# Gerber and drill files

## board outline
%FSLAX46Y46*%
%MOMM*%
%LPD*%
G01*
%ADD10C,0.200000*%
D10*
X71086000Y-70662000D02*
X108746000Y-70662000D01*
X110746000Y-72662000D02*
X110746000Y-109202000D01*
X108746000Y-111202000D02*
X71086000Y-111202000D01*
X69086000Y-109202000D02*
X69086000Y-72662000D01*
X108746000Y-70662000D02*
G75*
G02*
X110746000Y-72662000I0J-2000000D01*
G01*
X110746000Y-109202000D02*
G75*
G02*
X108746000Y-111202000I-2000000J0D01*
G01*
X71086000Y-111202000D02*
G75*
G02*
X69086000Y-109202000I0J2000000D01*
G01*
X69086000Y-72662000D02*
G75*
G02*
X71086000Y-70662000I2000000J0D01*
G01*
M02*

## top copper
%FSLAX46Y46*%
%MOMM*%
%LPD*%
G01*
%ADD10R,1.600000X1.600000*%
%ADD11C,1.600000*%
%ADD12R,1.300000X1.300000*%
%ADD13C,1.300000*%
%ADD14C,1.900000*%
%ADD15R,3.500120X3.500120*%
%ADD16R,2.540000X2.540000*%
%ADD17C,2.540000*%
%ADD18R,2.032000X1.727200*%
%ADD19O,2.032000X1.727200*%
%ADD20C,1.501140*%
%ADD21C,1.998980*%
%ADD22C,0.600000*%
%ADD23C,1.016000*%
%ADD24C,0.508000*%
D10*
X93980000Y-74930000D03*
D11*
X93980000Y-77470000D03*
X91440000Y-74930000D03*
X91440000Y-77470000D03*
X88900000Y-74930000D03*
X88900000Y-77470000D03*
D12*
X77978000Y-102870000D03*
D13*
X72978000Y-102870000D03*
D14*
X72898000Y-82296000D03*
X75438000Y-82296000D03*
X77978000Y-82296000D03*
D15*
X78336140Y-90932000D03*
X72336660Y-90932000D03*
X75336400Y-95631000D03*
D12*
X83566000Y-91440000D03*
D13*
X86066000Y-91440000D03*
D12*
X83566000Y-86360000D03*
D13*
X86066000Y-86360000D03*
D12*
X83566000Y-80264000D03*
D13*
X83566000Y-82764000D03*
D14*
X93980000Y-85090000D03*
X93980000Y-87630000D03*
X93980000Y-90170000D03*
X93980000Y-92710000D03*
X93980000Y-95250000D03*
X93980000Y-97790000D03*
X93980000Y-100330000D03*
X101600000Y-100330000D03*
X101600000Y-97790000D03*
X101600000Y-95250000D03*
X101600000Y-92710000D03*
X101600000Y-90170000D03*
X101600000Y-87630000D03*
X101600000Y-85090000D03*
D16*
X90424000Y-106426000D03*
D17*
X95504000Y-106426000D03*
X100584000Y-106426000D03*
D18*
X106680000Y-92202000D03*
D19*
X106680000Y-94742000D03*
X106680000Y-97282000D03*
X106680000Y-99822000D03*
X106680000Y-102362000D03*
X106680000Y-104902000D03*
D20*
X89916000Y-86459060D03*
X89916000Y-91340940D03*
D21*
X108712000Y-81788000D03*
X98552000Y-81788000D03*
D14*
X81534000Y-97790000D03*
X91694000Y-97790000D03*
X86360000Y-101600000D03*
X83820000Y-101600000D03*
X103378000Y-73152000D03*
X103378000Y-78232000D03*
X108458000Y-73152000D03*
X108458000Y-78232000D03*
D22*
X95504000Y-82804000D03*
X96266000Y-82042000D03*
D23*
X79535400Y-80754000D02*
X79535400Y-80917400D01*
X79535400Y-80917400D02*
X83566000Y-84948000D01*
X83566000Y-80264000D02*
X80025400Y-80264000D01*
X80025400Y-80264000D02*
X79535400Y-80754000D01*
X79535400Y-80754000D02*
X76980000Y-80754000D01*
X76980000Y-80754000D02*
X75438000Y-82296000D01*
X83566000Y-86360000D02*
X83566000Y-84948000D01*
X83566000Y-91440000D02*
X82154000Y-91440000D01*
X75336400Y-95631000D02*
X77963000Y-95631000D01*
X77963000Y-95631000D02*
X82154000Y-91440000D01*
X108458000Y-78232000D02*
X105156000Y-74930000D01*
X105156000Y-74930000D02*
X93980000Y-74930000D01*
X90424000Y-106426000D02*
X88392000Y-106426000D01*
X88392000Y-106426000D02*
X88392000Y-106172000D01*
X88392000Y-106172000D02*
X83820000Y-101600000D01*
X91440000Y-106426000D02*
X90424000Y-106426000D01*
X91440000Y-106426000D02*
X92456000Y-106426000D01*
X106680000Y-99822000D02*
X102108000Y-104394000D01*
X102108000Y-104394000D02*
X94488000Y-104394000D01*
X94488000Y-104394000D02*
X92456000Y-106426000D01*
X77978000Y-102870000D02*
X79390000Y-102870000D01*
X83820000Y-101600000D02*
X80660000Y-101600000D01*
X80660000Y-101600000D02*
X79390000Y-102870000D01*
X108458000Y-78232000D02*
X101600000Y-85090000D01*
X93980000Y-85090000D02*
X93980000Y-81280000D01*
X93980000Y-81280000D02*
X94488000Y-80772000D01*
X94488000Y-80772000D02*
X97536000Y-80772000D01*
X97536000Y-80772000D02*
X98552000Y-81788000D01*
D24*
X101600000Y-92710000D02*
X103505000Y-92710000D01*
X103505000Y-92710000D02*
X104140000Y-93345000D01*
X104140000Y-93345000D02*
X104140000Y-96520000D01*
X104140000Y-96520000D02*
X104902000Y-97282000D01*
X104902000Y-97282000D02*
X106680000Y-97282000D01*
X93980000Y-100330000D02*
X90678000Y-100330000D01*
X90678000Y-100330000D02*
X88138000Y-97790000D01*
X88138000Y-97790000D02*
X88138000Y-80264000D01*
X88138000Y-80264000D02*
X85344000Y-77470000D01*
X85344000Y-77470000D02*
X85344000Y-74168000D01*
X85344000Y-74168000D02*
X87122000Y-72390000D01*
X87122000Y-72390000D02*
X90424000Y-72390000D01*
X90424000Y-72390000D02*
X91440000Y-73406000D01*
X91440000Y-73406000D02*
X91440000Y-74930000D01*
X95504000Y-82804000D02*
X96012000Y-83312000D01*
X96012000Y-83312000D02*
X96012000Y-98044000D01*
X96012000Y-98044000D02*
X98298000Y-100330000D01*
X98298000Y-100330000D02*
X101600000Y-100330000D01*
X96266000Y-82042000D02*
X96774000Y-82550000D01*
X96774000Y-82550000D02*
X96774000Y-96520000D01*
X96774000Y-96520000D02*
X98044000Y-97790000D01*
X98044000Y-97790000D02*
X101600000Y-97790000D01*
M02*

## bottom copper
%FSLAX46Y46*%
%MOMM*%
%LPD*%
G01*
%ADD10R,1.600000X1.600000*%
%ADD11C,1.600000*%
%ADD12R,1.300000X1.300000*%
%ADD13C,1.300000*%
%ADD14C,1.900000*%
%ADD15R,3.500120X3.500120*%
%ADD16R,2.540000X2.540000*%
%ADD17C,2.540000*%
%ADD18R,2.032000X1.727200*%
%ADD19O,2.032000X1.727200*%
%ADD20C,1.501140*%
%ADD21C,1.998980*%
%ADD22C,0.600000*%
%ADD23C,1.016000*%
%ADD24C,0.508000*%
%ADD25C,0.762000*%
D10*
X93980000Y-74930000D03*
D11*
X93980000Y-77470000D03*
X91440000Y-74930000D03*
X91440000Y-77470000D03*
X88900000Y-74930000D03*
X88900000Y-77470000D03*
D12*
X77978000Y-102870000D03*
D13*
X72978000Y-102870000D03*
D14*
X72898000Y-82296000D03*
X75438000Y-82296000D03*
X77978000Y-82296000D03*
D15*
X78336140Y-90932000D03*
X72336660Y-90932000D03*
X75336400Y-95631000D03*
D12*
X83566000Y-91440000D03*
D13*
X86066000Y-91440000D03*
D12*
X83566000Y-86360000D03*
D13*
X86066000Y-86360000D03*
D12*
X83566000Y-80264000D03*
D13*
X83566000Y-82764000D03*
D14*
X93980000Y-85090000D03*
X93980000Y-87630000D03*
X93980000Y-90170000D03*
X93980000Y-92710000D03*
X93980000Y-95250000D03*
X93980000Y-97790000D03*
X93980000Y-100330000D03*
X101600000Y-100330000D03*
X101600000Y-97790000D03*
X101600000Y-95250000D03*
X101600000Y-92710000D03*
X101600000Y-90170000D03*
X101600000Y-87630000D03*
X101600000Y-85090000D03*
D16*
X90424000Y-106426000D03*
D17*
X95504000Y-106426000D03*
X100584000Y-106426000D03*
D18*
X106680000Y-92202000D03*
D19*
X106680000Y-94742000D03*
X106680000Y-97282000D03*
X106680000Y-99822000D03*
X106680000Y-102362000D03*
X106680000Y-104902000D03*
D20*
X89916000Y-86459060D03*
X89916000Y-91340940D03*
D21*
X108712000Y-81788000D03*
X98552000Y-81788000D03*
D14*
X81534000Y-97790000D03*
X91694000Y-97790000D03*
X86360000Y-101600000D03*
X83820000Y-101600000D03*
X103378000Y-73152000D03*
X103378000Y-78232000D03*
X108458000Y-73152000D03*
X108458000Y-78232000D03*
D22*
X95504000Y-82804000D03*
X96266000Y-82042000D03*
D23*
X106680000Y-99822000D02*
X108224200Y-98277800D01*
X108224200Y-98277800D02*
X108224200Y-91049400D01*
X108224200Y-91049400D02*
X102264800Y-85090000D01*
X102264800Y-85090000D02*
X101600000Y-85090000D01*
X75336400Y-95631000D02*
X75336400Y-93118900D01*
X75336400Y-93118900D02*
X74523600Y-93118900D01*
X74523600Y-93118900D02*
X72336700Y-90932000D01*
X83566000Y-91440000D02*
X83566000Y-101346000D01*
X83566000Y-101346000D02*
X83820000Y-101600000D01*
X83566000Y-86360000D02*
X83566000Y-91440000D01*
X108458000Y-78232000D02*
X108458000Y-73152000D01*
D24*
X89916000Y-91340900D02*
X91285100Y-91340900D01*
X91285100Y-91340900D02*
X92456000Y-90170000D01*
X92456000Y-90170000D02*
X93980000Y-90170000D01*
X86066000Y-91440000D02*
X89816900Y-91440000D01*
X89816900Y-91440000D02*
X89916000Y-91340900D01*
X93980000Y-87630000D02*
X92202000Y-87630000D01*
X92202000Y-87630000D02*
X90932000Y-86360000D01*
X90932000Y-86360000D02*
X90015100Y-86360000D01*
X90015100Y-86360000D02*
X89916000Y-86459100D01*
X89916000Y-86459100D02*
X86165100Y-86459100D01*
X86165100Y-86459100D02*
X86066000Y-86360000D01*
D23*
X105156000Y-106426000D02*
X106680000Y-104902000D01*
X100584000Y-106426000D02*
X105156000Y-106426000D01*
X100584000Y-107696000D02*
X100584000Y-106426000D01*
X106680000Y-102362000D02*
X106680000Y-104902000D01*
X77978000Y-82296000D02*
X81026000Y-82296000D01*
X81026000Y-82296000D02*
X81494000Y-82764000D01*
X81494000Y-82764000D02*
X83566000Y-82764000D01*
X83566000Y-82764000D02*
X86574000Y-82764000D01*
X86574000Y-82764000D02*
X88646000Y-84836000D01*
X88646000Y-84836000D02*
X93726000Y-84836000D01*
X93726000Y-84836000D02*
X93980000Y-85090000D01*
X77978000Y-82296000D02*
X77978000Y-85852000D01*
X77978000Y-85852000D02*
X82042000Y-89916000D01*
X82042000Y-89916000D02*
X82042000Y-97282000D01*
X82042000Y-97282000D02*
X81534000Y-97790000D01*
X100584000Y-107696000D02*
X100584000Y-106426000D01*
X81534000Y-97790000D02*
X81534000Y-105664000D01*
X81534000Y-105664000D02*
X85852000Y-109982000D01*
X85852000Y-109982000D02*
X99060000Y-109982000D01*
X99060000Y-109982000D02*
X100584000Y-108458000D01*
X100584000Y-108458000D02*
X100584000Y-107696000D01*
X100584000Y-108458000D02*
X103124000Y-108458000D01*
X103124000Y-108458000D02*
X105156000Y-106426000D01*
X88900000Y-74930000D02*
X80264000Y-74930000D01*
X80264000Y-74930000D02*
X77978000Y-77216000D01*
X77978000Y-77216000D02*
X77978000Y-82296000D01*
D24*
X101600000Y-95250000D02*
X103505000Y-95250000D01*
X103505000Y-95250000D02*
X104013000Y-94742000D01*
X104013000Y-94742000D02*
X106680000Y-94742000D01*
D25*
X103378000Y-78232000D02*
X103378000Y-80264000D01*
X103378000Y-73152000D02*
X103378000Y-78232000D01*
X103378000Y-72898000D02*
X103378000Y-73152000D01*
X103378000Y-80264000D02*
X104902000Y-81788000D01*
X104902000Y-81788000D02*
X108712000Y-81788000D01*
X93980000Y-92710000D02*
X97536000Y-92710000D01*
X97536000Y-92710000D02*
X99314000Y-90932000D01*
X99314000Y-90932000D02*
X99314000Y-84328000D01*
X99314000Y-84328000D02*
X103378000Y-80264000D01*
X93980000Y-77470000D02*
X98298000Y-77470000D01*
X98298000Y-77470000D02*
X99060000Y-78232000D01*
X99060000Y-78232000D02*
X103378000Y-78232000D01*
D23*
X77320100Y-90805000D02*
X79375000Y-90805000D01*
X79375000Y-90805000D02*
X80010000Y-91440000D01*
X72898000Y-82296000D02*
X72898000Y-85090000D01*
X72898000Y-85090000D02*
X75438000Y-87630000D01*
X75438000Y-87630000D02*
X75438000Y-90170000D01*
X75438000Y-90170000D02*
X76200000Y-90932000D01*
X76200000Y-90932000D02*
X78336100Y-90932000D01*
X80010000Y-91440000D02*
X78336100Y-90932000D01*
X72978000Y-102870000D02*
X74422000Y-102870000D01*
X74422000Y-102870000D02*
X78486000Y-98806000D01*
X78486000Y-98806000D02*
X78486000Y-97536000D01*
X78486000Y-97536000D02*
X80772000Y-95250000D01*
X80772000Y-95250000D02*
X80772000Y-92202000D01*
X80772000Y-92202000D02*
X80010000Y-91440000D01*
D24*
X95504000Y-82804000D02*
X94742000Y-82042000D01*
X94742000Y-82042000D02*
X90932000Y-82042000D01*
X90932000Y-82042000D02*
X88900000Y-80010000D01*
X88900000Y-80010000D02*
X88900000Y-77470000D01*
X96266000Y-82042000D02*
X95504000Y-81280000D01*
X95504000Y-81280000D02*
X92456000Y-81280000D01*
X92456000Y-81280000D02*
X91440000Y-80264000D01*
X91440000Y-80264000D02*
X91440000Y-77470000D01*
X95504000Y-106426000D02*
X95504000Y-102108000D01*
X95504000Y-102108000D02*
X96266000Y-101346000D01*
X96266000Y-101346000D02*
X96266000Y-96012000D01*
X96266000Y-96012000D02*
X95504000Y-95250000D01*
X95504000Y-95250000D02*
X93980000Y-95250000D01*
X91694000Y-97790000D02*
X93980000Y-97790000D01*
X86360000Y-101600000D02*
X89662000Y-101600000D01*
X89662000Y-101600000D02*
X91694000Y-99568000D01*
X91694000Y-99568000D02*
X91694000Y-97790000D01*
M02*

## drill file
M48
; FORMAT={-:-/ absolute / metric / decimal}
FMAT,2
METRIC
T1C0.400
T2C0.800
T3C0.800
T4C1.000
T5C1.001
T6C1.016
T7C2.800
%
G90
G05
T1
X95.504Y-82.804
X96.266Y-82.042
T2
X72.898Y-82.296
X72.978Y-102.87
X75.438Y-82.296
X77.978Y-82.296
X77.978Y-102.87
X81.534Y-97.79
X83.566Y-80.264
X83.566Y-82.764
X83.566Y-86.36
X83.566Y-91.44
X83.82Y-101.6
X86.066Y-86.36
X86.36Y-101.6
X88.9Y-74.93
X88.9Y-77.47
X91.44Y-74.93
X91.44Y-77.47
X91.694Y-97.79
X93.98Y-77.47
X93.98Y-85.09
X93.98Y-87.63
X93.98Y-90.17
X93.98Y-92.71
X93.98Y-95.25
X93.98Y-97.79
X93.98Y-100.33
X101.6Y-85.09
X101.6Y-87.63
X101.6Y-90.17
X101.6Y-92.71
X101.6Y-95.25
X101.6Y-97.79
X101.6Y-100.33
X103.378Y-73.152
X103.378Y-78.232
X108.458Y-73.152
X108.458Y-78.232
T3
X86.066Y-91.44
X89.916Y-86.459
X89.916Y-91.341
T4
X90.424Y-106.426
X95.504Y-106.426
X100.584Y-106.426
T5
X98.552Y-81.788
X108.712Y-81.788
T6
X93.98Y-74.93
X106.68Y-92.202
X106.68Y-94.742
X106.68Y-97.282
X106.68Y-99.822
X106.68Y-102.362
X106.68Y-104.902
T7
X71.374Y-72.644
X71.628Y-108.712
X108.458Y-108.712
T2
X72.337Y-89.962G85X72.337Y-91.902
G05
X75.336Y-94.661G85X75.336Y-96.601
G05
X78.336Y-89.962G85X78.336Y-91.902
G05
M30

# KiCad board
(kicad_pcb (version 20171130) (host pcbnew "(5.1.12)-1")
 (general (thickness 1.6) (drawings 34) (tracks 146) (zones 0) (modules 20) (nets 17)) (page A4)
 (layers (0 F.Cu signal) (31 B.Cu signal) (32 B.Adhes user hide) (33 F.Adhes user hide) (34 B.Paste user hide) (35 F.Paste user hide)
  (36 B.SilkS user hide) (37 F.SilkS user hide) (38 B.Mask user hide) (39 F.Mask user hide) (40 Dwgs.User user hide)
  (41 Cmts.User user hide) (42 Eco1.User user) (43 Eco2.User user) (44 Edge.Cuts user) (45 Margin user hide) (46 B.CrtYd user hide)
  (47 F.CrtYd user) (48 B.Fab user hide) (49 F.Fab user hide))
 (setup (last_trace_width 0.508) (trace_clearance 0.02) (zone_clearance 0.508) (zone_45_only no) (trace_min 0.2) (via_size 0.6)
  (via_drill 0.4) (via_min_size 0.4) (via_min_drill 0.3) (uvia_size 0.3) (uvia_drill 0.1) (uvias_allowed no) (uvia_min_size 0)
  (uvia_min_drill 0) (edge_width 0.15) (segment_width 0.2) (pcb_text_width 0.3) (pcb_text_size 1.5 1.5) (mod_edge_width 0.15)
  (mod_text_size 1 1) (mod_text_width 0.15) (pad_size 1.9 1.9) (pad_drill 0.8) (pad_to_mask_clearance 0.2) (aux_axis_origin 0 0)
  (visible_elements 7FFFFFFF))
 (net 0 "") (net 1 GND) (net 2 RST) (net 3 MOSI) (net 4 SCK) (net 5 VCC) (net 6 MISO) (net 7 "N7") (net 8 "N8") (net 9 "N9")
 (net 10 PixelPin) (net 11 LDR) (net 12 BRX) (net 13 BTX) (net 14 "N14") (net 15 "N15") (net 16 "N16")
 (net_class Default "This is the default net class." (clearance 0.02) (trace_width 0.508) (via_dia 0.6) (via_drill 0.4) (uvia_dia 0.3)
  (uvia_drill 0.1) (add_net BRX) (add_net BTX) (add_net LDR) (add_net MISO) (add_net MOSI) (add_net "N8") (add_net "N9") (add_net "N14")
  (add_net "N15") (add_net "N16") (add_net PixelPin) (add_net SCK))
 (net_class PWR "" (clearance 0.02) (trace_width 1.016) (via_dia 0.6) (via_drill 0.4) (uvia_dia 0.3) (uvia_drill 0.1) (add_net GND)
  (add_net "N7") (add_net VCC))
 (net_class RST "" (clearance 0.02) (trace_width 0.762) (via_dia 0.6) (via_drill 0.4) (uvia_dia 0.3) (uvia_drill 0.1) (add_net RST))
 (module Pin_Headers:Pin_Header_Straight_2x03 (layer F.Cu) (at 93.98 74.93 270)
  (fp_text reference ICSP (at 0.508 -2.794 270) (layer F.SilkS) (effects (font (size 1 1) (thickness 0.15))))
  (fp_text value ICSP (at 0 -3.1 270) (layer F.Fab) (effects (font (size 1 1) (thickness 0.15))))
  (pad 1 thru_hole rect (at 0 0 270) (size 1.6 1.6) (drill 1.016) (layers *.Cu *.Mask F.SilkS) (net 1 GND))
  (pad 2 thru_hole circle (at 2.54 0 270) (size 1.6 1.6) (drill 0.8) (layers *.Cu *.Mask F.SilkS) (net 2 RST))
  (pad 3 thru_hole circle (at 0 2.54 270) (size 1.6 1.6) (drill 0.8) (layers *.Cu *.Mask F.SilkS) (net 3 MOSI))
  (pad 4 thru_hole circle (at 2.54 2.54 270) (size 1.6 1.6) (drill 0.8) (layers *.Cu *.Mask F.SilkS) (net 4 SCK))
  (pad 5 thru_hole circle (at 0 5.08 270) (size 1.6 1.6) (drill 0.8) (layers *.Cu *.Mask F.SilkS) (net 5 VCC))
  (pad 6 thru_hole circle (at 2.54 5.08 270) (size 1.6 1.6) (drill 0.8) (layers *.Cu *.Mask F.SilkS) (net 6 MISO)))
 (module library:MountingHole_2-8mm (layer F.Cu) (at 71.628 108.712)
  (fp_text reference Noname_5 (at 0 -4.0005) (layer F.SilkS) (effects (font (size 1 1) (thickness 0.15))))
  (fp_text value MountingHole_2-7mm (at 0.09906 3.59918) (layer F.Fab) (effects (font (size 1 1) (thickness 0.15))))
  (pad "" np_thru_hole circle (at 0 0) (size 2.8 2.8) (drill 2.8) (layers *.Cu *.Mask F.SilkS)))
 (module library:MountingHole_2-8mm (layer F.Cu) (at 71.374 72.644)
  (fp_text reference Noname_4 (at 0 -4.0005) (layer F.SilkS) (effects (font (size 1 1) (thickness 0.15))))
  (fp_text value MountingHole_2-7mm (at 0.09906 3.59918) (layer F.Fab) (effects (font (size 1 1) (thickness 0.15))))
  (pad "" np_thru_hole circle (at 0 0) (size 2.8 2.8) (drill 2.8) (layers *.Cu *.Mask F.SilkS)))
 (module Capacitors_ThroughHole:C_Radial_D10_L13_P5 (layer F.Cu) (at 77.978 102.87 180)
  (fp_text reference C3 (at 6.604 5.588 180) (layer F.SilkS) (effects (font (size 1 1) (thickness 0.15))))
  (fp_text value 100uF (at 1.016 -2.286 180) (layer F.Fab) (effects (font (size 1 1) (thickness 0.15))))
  (pad 1 thru_hole rect (at 0 0 180) (size 1.3 1.3) (drill 0.8) (layers *.Cu *.Mask F.SilkS) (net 1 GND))
  (pad 2 thru_hole circle (at 5 0 180) (size 1.3 1.3) (drill 0.8) (layers *.Cu *.Mask F.SilkS) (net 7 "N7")))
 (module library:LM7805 (layer F.Cu) (at 72.898 82.296)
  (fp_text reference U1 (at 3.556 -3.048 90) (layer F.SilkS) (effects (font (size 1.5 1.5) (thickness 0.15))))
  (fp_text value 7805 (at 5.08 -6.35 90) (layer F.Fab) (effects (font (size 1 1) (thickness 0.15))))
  (pad VI thru_hole circle (at 0 0) (size 1.9 1.9) (drill 0.8) (layers *.Cu *.Mask F.SilkS) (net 7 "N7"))
  (pad GND thru_hole circle (at 2.54 0) (size 1.9 1.9) (drill 0.8) (layers *.Cu *.Mask F.SilkS) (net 1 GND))
  (pad VO thru_hole circle (at 5.08 0) (size 1.9 1.9) (drill 0.8) (layers *.Cu *.Mask F.SilkS) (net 5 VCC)))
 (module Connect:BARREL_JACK (layer F.Cu) (at 72.136 90.932)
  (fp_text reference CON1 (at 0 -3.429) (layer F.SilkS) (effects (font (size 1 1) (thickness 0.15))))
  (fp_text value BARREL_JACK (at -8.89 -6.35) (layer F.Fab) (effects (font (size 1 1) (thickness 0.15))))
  (pad 1 thru_hole rect (at 6.20014 0) (size 3.50012 3.50012) (drill oval 0.8 2.74) (layers *.Cu *.Mask F.SilkS) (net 7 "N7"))
  (pad 2 thru_hole rect (at 0.20066 0) (size 3.50012 3.50012) (drill oval 0.8 2.74) (layers *.Cu *.Mask F.SilkS) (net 1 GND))
  (pad 3 thru_hole rect (at 3.2004 4.699) (size 3.50012 3.50012) (drill oval 0.8 2.74) (layers *.Cu *.Mask F.SilkS) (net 1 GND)))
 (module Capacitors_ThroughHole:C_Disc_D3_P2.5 (layer F.Cu) (at 83.566 91.44)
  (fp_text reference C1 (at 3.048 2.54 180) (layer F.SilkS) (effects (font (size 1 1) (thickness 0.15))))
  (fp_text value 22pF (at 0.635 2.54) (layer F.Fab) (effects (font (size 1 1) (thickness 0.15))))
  (pad 1 thru_hole rect (at 0 0) (size 1.3 1.3) (drill 0.8) (layers *.Cu *.Mask F.SilkS) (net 1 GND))
  (pad 2 thru_hole circle (at 2.5 0) (size 1.3 1.3) (drill 0.8001) (layers *.Cu *.Mask F.SilkS) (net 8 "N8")))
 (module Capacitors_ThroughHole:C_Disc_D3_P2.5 (layer F.Cu) (at 83.566 86.36)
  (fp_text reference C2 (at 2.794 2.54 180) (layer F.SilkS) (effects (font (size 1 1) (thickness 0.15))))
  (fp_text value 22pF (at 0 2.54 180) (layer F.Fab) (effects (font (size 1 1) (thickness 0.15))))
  (pad 1 thru_hole rect (at 0 0) (size 1.3 1.3) (drill 0.8) (layers *.Cu *.Mask F.SilkS) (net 1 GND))
  (pad 2 thru_hole circle (at 2.5 0) (size 1.3 1.3) (drill 0.8) (layers *.Cu *.Mask F.SilkS) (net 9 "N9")))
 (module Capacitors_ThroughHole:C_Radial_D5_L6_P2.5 (layer F.Cu) (at 83.566 80.264 270)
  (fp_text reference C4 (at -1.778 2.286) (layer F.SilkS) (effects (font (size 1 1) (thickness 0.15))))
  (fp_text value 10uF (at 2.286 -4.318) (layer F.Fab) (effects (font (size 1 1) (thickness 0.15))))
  (pad 1 thru_hole rect (at 0 0 270) (size 1.3 1.3) (drill 0.8) (layers *.Cu *.Mask F.SilkS) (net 1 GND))
  (pad 2 thru_hole circle (at 2.5 0 270) (size 1.3 1.3) (drill 0.8) (layers *.Cu *.Mask F.SilkS) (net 5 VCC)))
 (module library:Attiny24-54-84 (layer F.Cu) (at 93.98 85.09)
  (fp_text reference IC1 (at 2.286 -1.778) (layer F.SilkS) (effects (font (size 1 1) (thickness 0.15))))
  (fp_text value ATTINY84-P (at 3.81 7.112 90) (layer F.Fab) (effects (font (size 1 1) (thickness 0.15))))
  (pad 1 thru_hole circle (at 0 0) (size 1.9 1.9) (drill 0.8) (layers *.Cu *.Mask F.SilkS) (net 5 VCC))
  (pad 2 thru_hole circle (at 0 2.54) (size 1.9 1.9) (drill 0.8) (layers *.Cu *.Mask F.SilkS) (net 9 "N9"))
  (pad 3 thru_hole circle (at 0 5.08) (size 1.9 1.9) (drill 0.8) (layers *.Cu *.Mask F.SilkS) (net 8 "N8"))
  (pad 4 thru_hole circle (at 0 7.62) (size 1.9 1.9) (drill 0.8) (layers *.Cu *.Mask F.SilkS) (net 2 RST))
  (pad 5 thru_hole circle (at 0 10.16) (size 1.9 1.9) (drill 0.8) (layers *.Cu *.Mask F.SilkS) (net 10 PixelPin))
  (pad 6 thru_hole circle (at 0 12.7) (size 1.9 1.9) (drill 0.8) (layers *.Cu *.Mask F.SilkS) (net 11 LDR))
  (pad 7 thru_hole circle (at 0 15.24) (size 1.9 1.9) (drill 0.8) (layers *.Cu *.Mask F.SilkS) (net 3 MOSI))
  (pad 8 thru_hole circle (at 7.62 15.24) (size 1.9 1.9) (drill 0.8) (layers *.Cu *.Mask F.SilkS) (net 6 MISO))
  (pad 9 thru_hole circle (at 7.62 12.7) (size 1.9 1.9) (drill 0.8) (layers *.Cu *.Mask F.SilkS) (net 4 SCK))
  (pad 10 thru_hole circle (at 7.62 10.16) (size 1.9 1.9) (drill 0.8) (layers *.Cu *.Mask F.SilkS) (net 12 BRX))
  (pad 11 thru_hole circle (at 7.62 7.62) (size 1.9 1.9) (drill 0.8) (layers *.Cu *.Mask F.SilkS) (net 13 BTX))
  (pad 12 thru_hole circle (at 7.62 5.08) (size 1.9 1.9) (drill 0.8) (layers *.Cu *.Mask F.SilkS) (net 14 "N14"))
  (pad 13 thru_hole circle (at 7.62 2.54) (size 1.9 1.9) (drill 0.8) (layers *.Cu *.Mask F.SilkS) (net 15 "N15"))
  (pad 14 thru_hole circle (at 7.62 0) (size 1.9 1.9) (drill 0.8) (layers *.Cu *.Mask F.SilkS) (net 1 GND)))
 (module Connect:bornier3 (layer F.Cu) (at 95.504 106.426)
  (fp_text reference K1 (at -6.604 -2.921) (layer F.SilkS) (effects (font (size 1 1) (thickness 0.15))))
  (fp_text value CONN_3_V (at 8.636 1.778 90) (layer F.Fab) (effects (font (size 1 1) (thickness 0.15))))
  (pad 1 thru_hole rect (at -5.08 0) (size 2.54 2.54) (drill 1) (layers *.Cu *.Mask F.SilkS) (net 1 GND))
  (pad 2 thru_hole circle (at 0 0) (size 2.54 2.54) (drill 1) (layers *.Cu *.Mask F.SilkS) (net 10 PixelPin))
  (pad 3 thru_hole circle (at 5.08 0) (size 2.54 2.54) (drill 1) (layers *.Cu *.Mask F.SilkS) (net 5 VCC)))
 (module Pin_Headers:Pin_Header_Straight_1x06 (layer F.Cu) (at 106.68 92.202)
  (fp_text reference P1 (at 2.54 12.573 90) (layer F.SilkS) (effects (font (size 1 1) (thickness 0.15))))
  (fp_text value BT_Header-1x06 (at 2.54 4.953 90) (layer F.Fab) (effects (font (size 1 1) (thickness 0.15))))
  (pad 1 thru_hole rect (at 0 0) (size 2.032 1.7272) (drill 1.016) (layers *.Cu *.Mask F.SilkS) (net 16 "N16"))
  (pad 2 thru_hole oval (at 0 2.54) (size 2.032 1.7272) (drill 1.016) (layers *.Cu *.Mask F.SilkS) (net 12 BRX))
  (pad 3 thru_hole oval (at 0 5.08) (size 2.032 1.7272) (drill 1.016) (layers *.Cu *.Mask F.SilkS) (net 13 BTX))
  (pad 4 thru_hole oval (at 0 7.62) (size 2.032 1.7272) (drill 1.016) (layers *.Cu *.Mask F.SilkS) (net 1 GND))
  (pad 5 thru_hole oval (at 0 10.16) (size 2.032 1.7272) (drill 1.016) (layers *.Cu *.Mask F.SilkS) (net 5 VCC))
  (pad 6 thru_hole oval (at 0 12.7) (size 2.032 1.7272) (drill 1.016) (layers *.Cu *.Mask F.SilkS) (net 5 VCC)))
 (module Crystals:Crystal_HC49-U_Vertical (layer F.Cu) (at 89.916 88.9 270)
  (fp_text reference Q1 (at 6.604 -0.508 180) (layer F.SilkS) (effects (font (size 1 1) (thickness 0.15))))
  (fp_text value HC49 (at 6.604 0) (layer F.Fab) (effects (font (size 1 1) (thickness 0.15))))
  (pad 1 thru_hole circle (at -2.44094 0 270) (size 1.50114 1.50114) (drill 0.8001) (layers *.Cu *.Mask F.SilkS) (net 9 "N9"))
  (pad 2 thru_hole circle (at 2.44094 0 270) (size 1.50114 1.50114) (drill 0.8001) (layers *.Cu *.Mask F.SilkS) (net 8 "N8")))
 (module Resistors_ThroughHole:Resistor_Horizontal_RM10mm (layer F.Cu) (at 103.632 81.788 180)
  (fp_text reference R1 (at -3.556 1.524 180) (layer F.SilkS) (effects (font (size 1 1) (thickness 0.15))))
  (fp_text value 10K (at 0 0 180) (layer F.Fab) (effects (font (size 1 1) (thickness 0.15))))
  (pad 1 thru_hole circle (at -5.08 0 180) (size 1.99898 1.99898) (drill 1.00076) (layers *.Cu *.SilkS *.Mask) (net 2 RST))
  (pad 2 thru_hole circle (at 5.08 0 180) (size 1.99898 1.99898) (drill 1.00076) (layers *.Cu *.SilkS *.Mask) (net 5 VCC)))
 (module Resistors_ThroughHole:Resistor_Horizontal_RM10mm (layer F.Cu) (at 86.614 97.79)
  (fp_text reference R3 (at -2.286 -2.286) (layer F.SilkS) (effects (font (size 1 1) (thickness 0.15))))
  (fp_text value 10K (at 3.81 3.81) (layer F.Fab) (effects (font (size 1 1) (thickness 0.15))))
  (pad 1 thru_hole circle (at -5.08 0) (size 1.9 1.9) (drill 0.8) (layers *.Cu *.Mask F.SilkS) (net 5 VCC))
  (pad 2 thru_hole circle (at 5.08 0) (size 1.9 1.9) (drill 0.8) (layers *.Cu *.Mask F.SilkS) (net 11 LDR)))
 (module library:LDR (layer F.Cu) (at 86.36 101.6 180)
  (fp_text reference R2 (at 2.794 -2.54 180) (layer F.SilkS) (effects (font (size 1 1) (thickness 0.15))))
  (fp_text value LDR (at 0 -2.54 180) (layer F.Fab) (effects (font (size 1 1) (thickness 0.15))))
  (pad 1 thru_hole circle (at 0 0 180) (size 1.9 1.9) (drill 0.8) (layers *.Cu *.Mask F.SilkS) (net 11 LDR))
  (pad 2 thru_hole circle (at 2.54 0 180) (size 1.9 1.9) (drill 0.8) (layers *.Cu *.Mask F.SilkS) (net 1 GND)))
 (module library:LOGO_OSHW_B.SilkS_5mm (layer F.Cu) (at 106.934 86.614)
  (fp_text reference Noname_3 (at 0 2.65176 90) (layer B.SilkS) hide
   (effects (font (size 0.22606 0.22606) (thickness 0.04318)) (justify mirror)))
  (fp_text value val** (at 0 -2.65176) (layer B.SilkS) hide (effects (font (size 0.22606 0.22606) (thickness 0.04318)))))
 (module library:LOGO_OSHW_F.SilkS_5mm (layer F.Cu) (at 106.934 86.614)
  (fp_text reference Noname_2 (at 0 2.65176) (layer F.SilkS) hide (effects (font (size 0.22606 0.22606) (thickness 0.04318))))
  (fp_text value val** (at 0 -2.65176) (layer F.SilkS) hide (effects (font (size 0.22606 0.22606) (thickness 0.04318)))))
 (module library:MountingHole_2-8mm (layer F.Cu) (at 108.458 108.712)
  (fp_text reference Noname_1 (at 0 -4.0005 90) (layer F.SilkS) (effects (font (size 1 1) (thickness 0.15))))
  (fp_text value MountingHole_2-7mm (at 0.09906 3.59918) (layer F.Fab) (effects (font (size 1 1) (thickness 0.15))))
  (pad "" np_thru_hole circle (at 0 0) (size 2.8 2.8) (drill 2.8) (layers *.Cu *.Mask F.SilkS)))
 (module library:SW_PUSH (layer F.Cu) (at 103.378 73.152)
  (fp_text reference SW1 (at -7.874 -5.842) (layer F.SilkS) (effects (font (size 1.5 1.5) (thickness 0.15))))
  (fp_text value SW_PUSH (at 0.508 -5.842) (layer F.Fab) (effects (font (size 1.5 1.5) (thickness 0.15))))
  (pad 1 thru_hole circle (at 0 0) (size 1.9 1.9) (drill 0.8) (layers *.Cu *.Mask F.SilkS) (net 2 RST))
  (pad 1 thru_hole circle (at 0 5.08) (size 1.9 1.9) (drill 0.8) (layers *.Cu *.Mask F.SilkS) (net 2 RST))
  (pad 2 thru_hole circle (at 5.08 0) (size 1.9 1.9) (drill 0.8) (layers *.Cu *.Mask F.SilkS) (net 1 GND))
  (pad 2 thru_hole circle (at 5.08 5.08) (size 1.9 1.9) (drill 0.8) (layers *.Cu *.Mask F.SilkS) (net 1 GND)))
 (gr_line (start 71.086 70.662) (end 108.746 70.662) (angle 90) (layer Edge.Cuts) (width 0.2))
 (gr_line (start 110.746 72.662) (end 110.746 109.202) (angle 90) (layer Edge.Cuts) (width 0.2))
 (gr_line (start 108.746 111.202) (end 71.086 111.202) (angle 90) (layer Edge.Cuts) (width 0.2))
 (gr_line (start 69.086 109.202) (end 69.086 72.662) (angle 90) (layer Edge.Cuts) (width 0.2))
 (gr_arc (start 108.746 72.662) (end 108.746 70.662) (angle 90) (layer Edge.Cuts) (width 0.2))
 (gr_arc (start 108.746 109.202) (end 110.746 109.202) (angle 90) (layer Edge.Cuts) (width 0.2))
 (gr_arc (start 71.086 109.202) (end 71.086 111.202) (angle 90) (layer Edge.Cuts) (width 0.2))
 (gr_arc (start 71.086 72.662) (end 69.086 72.662) (angle 90) (layer Edge.Cuts) (width 0.2))
 (segment (start 106.68 99.822) (end 108.2242 98.2778) (width 1.016) (layer B.Cu) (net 1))
 (segment (start 108.2242 98.2778) (end 108.2242 91.0494) (width 1.016) (layer B.Cu) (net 1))
 (segment (start 108.2242 91.0494) (end 102.2648 85.09) (width 1.016) (layer B.Cu) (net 1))
 (segment (start 102.2648 85.09) (end 101.6 85.09) (width 1.016) (layer B.Cu) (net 1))
 (segment (start 79.5354 80.754) (end 79.5354 80.9174) (width 1.016) (layer F.Cu) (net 1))
 (segment (start 79.5354 80.9174) (end 83.566 84.948) (width 1.016) (layer F.Cu) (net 1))
 (segment (start 83.566 80.264) (end 80.0254 80.264) (width 1.016) (layer F.Cu) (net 1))
 (segment (start 80.0254 80.264) (end 79.5354 80.754) (width 1.016) (layer F.Cu) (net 1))
 (segment (start 79.5354 80.754) (end 76.98 80.754) (width 1.016) (layer F.Cu) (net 1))
 (segment (start 76.98 80.754) (end 75.438 82.296) (width 1.016) (layer F.Cu) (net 1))
 (segment (start 83.566 86.36) (end 83.566 84.948) (width 1.016) (layer F.Cu) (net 1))
 (segment (start 83.566 91.44) (end 82.154 91.44) (width 1.016) (layer F.Cu) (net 1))
 (segment (start 75.3364 95.631) (end 77.963 95.631) (width 1.016) (layer F.Cu) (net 1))
 (segment (start 77.963 95.631) (end 82.154 91.44) (width 1.016) (layer F.Cu) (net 1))
 (segment (start 75.3364 95.631) (end 75.3364 93.1189) (width 1.016) (layer B.Cu) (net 1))
 (segment (start 75.3364 93.1189) (end 74.5236 93.1189) (width 1.016) (layer B.Cu) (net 1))
 (segment (start 74.5236 93.1189) (end 72.3367 90.932) (width 1.016) (layer B.Cu) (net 1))
 (segment (start 83.566 91.44) (end 83.566 101.346) (width 1.016) (layer B.Cu) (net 1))
 (segment (start 83.566 101.346) (end 83.82 101.6) (width 1.016) (layer B.Cu) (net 1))
 (segment (start 83.566 86.36) (end 83.566 91.44) (width 1.016) (layer B.Cu) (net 1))
 (segment (start 108.458 78.232) (end 105.156 74.93) (width 1.016) (layer F.Cu) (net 1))
 (segment (start 105.156 74.93) (end 93.98 74.93) (width 1.016) (layer F.Cu) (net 1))
 (segment (start 90.424 106.426) (end 88.392 106.426) (width 1.016) (layer F.Cu) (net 1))
 (segment (start 88.392 106.426) (end 88.392 106.172) (width 1.016) (layer F.Cu) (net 1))
 (segment (start 88.392 106.172) (end 83.82 101.6) (width 1.016) (layer F.Cu) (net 1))
 (segment (start 91.44 106.426) (end 90.424 106.426) (width 1.016) (layer F.Cu) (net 1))
 (segment (start 91.44 106.426) (end 92.456 106.426) (width 1.016) (layer F.Cu) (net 1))
 (segment (start 106.68 99.822) (end 102.108 104.394) (width 1.016) (layer F.Cu) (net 1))
 (segment (start 102.108 104.394) (end 94.488 104.394) (width 1.016) (layer F.Cu) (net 1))
 (segment (start 94.488 104.394) (end 92.456 106.426) (width 1.016) (layer F.Cu) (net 1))
 (segment (start 77.978 102.87) (end 79.39 102.87) (width 1.016) (layer F.Cu) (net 1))
 (segment (start 83.82 101.6) (end 80.66 101.6) (width 1.016) (layer F.Cu) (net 1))
 (segment (start 80.66 101.6) (end 79.39 102.87) (width 1.016) (layer F.Cu) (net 1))
 (segment (start 108.458 78.232) (end 101.6 85.09) (width 1.016) (layer F.Cu) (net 1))
 (segment (start 108.458 78.232) (end 108.458 73.152) (width 1.016) (layer B.Cu) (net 1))
 (segment (start 89.916 91.3409) (end 91.2851 91.3409) (width 0.508) (layer B.Cu) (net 8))
 (segment (start 91.2851 91.3409) (end 92.456 90.17) (width 0.508) (layer B.Cu) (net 8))
 (segment (start 92.456 90.17) (end 93.98 90.17) (width 0.508) (layer B.Cu) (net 8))
 (segment (start 86.066 91.44) (end 89.8169 91.44) (width 0.508) (layer B.Cu) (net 8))
 (segment (start 89.8169 91.44) (end 89.916 91.3409) (width 0.508) (layer B.Cu) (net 8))
 (segment (start 93.98 87.63) (end 92.202 87.63) (width 0.508) (layer B.Cu) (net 9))
 (segment (start 92.202 87.63) (end 90.932 86.36) (width 0.508) (layer B.Cu) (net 9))
 (segment (start 90.932 86.36) (end 90.0151 86.36) (width 0.508) (layer B.Cu) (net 9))
 (segment (start 90.0151 86.36) (end 89.916 86.4591) (width 0.508) (layer B.Cu) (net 9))
 (segment (start 89.916 86.4591) (end 86.1651 86.4591) (width 0.508) (layer B.Cu) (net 9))
 (segment (start 86.1651 86.4591) (end 86.066 86.36) (width 0.508) (layer B.Cu) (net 9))
 (segment (start 105.156 106.426) (end 106.68 104.902) (width 1.016) (layer B.Cu) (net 5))
 (segment (start 100.584 106.426) (end 105.156 106.426) (width 1.016) (layer B.Cu) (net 5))
 (segment (start 100.584 107.696) (end 100.584 106.426) (width 1.016) (layer B.Cu) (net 5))
 (segment (start 106.68 102.362) (end 106.68 104.902) (width 1.016) (layer B.Cu) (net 5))
 (segment (start 77.978 82.296) (end 81.026 82.296) (width 1.016) (layer B.Cu) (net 5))
 (segment (start 81.026 82.296) (end 81.494 82.764) (width 1.016) (layer B.Cu) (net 5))
 (segment (start 81.494 82.764) (end 83.566 82.764) (width 1.016) (layer B.Cu) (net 5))
 (segment (start 83.566 82.764) (end 86.574 82.764) (width 1.016) (layer B.Cu) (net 5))
 (segment (start 86.574 82.764) (end 88.646 84.836) (width 1.016) (layer B.Cu) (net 5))
 (segment (start 88.646 84.836) (end 93.726 84.836) (width 1.016) (layer B.Cu) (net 5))
 (segment (start 93.726 84.836) (end 93.98 85.09) (width 1.016) (layer B.Cu) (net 5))
 (segment (start 93.98 85.09) (end 93.98 81.28) (width 1.016) (layer F.Cu) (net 5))
 (segment (start 93.98 81.28) (end 94.488 80.772) (width 1.016) (layer F.Cu) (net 5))
 (segment (start 94.488 80.772) (end 97.536 80.772) (width 1.016) (layer F.Cu) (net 5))
 (segment (start 97.536 80.772) (end 98.552 81.788) (width 1.016) (layer F.Cu) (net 5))
 (segment (start 77.978 82.296) (end 77.978 85.852) (width 1.016) (layer B.Cu) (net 5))
 (segment (start 77.978 85.852) (end 82.042 89.916) (width 1.016) (layer B.Cu) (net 5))
 (segment (start 82.042 89.916) (end 82.042 97.282) (width 1.016) (layer B.Cu) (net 5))
 (segment (start 82.042 97.282) (end 81.534 97.79) (width 1.016) (layer B.Cu) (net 5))
 (segment (start 100.584 107.696) (end 100.584 106.426) (width 1.016) (layer B.Cu) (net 5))
 (segment (start 81.534 97.79) (end 81.534 105.664) (width 1.016) (layer B.Cu) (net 5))
 (segment (start 81.534 105.664) (end 85.852 109.982) (width 1.016) (layer B.Cu) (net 5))
 (segment (start 85.852 109.982) (end 99.06 109.982) (width 1.016) (layer B.Cu) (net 5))
 (segment (start 99.06 109.982) (end 100.584 108.458) (width 1.016) (layer B.Cu) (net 5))
 (segment (start 100.584 108.458) (end 100.584 107.696) (width 1.016) (layer B.Cu) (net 5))
 (segment (start 100.584 108.458) (end 103.124 108.458) (width 1.016) (layer B.Cu) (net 5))
 (segment (start 103.124 108.458) (end 105.156 106.426) (width 1.016) (layer B.Cu) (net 5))
 (segment (start 88.9 74.93) (end 80.264 74.93) (width 1.016) (layer B.Cu) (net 5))
 (segment (start 80.264 74.93) (end 77.978 77.216) (width 1.016) (layer B.Cu) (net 5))
 (segment (start 77.978 77.216) (end 77.978 82.296) (width 1.016) (layer B.Cu) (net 5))
 (segment (start 101.6 95.25) (end 103.505 95.25) (width 0.508) (layer B.Cu) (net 12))
 (segment (start 103.505 95.25) (end 104.013 94.742) (width 0.508) (layer B.Cu) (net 12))
 (segment (start 104.013 94.742) (end 106.68 94.742) (width 0.508) (layer B.Cu) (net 12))
 (segment (start 101.6 92.71) (end 103.505 92.71) (width 0.508) (layer F.Cu) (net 13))
 (segment (start 103.505 92.71) (end 104.14 93.345) (width 0.508) (layer F.Cu) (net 13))
 (segment (start 104.14 93.345) (end 104.14 96.52) (width 0.508) (layer F.Cu) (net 13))
 (segment (start 104.14 96.52) (end 104.902 97.282) (width 0.508) (layer F.Cu) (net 13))
 (segment (start 104.902 97.282) (end 106.68 97.282) (width 0.508) (layer F.Cu) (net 13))
 (segment (start 103.378 78.232) (end 103.378 80.264) (width 0.762) (layer B.Cu) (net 2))
 (segment (start 103.378 73.152) (end 103.378 78.232) (width 0.762) (layer B.Cu) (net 2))
 (segment (start 103.378 72.898) (end 103.378 73.152) (width 0.762) (layer B.Cu) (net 2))
 (segment (start 103.378 80.264) (end 104.902 81.788) (width 0.762) (layer B.Cu) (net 2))
 (segment (start 104.902 81.788) (end 108.712 81.788) (width 0.762) (layer B.Cu) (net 2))
 (segment (start 93.98 92.71) (end 97.536 92.71) (width 0.762) (layer B.Cu) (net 2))
 (segment (start 97.536 92.71) (end 99.314 90.932) (width 0.762) (layer B.Cu) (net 2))
 (segment (start 99.314 90.932) (end 99.314 84.328) (width 0.762) (layer B.Cu) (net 2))
 (segment (start 99.314 84.328) (end 103.378 80.264) (width 0.762) (layer B.Cu) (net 2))
 (segment (start 93.98 77.47) (end 98.298 77.47) (width 0.762) (layer B.Cu) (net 2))
 (segment (start 98.298 77.47) (end 99.06 78.232) (width 0.762) (layer B.Cu) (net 2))
 (segment (start 99.06 78.232) (end 103.378 78.232) (width 0.762) (layer B.Cu) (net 2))
 (segment (start 77.3201 90.805) (end 79.375 90.805) (width 1.016) (layer B.Cu) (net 7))
 (segment (start 79.375 90.805) (end 80.01 91.44) (width 1.016) (layer B.Cu) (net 7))
 (segment (start 72.898 82.296) (end 72.898 85.09) (width 1.016) (layer B.Cu) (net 7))
 (segment (start 72.898 85.09) (end 75.438 87.63) (width 1.016) (layer B.Cu) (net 7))
 (segment (start 75.438 87.63) (end 75.438 90.17) (width 1.016) (layer B.Cu) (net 7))
 (segment (start 75.438 90.17) (end 76.2 90.932) (width 1.016) (layer B.Cu) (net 7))
 (segment (start 76.2 90.932) (end 78.3361 90.932) (width 1.016) (layer B.Cu) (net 7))
 (segment (start 80.01 91.44) (end 78.3361 90.932) (width 1.016) (layer B.Cu) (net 7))
 (segment (start 72.978 102.87) (end 74.422 102.87) (width 1.016) (layer B.Cu) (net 7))
 (segment (start 74.422 102.87) (end 78.486 98.806) (width 1.016) (layer B.Cu) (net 7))
 (segment (start 78.486 98.806) (end 78.486 97.536) (width 1.016) (layer B.Cu) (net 7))
 (segment (start 78.486 97.536) (end 80.772 95.25) (width 1.016) (layer B.Cu) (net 7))
 (segment (start 80.772 95.25) (end 80.772 92.202) (width 1.016) (layer B.Cu) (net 7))
 (segment (start 80.772 92.202) (end 80.01 91.44) (width 1.016) (layer B.Cu) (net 7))
 (segment (start 93.98 100.33) (end 90.678 100.33) (width 0.508) (layer F.Cu) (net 3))
 (segment (start 90.678 100.33) (end 88.138 97.79) (width 0.508) (layer F.Cu) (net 3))
 (segment (start 88.138 97.79) (end 88.138 80.264) (width 0.508) (layer F.Cu) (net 3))
 (segment (start 88.138 80.264) (end 85.344 77.47) (width 0.508) (layer F.Cu) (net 3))
 (segment (start 85.344 77.47) (end 85.344 74.168) (width 0.508) (layer F.Cu) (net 3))
 (segment (start 85.344 74.168) (end 87.122 72.39) (width 0.508) (layer F.Cu) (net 3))
 (segment (start 87.122 72.39) (end 90.424 72.39) (width 0.508) (layer F.Cu) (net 3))
 (segment (start 90.424 72.39) (end 91.44 73.406) (width 0.508) (layer F.Cu) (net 3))
 (segment (start 91.44 73.406) (end 91.44 74.93) (width 0.508) (layer F.Cu) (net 3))
 (segment (start 95.504 82.804) (end 96.012 83.312) (width 0.508) (layer F.Cu) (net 6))
 (segment (start 96.012 83.312) (end 96.012 98.044) (width 0.508) (layer F.Cu) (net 6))
 (segment (start 96.012 98.044) (end 98.298 100.33) (width 0.508) (layer F.Cu) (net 6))
 (segment (start 98.298 100.33) (end 101.6 100.33) (width 0.508) (layer F.Cu) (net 6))
 (segment (start 95.504 82.804) (end 94.742 82.042) (width 0.508) (layer B.Cu) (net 6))
 (segment (start 94.742 82.042) (end 90.932 82.042) (width 0.508) (layer B.Cu) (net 6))
 (segment (start 90.932 82.042) (end 88.9 80.01) (width 0.508) (layer B.Cu) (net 6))
 (segment (start 88.9 80.01) (end 88.9 77.47) (width 0.508) (layer B.Cu) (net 6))
 (via (at 95.504 82.804) (size 0.6) (layers F.Cu B.Cu) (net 6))
 (segment (start 96.266 82.042) (end 96.774 82.55) (width 0.508) (layer F.Cu) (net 4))
 (segment (start 96.774 82.55) (end 96.774 96.52) (width 0.508) (layer F.Cu) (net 4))
 (segment (start 96.774 96.52) (end 98.044 97.79) (width 0.508) (layer F.Cu) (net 4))
 (segment (start 98.044 97.79) (end 101.6 97.79) (width 0.508) (layer F.Cu) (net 4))
 (segment (start 96.266 82.042) (end 95.504 81.28) (width 0.508) (layer B.Cu) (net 4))
 (segment (start 95.504 81.28) (end 92.456 81.28) (width 0.508) (layer B.Cu) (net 4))
 (segment (start 92.456 81.28) (end 91.44 80.264) (width 0.508) (layer B.Cu) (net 4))
 (segment (start 91.44 80.264) (end 91.44 77.47) (width 0.508) (layer B.Cu) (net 4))
 (via (at 96.266 82.042) (size 0.6) (layers F.Cu B.Cu) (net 4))
 (segment (start 95.504 106.426) (end 95.504 102.108) (width 0.508) (layer B.Cu) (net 10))
 (segment (start 95.504 102.108) (end 96.266 101.346) (width 0.508) (layer B.Cu) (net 10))
 (segment (start 96.266 101.346) (end 96.266 96.012) (width 0.508) (layer B.Cu) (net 10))
 (segment (start 96.266 96.012) (end 95.504 95.25) (width 0.508) (layer B.Cu) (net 10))
 (segment (start 95.504 95.25) (end 93.98 95.25) (width 0.508) (layer B.Cu) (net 10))
 (segment (start 91.694 97.79) (end 93.98 97.79) (width 0.508) (layer B.Cu) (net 11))
 (segment (start 86.36 101.6) (end 89.662 101.6) (width 0.508) (layer B.Cu) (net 11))
 (segment (start 89.662 101.6) (end 91.694 99.568) (width 0.508) (layer B.Cu) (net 11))
 (segment (start 91.694 99.568) (end 91.694 97.79) (width 0.508) (layer B.Cu) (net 11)))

